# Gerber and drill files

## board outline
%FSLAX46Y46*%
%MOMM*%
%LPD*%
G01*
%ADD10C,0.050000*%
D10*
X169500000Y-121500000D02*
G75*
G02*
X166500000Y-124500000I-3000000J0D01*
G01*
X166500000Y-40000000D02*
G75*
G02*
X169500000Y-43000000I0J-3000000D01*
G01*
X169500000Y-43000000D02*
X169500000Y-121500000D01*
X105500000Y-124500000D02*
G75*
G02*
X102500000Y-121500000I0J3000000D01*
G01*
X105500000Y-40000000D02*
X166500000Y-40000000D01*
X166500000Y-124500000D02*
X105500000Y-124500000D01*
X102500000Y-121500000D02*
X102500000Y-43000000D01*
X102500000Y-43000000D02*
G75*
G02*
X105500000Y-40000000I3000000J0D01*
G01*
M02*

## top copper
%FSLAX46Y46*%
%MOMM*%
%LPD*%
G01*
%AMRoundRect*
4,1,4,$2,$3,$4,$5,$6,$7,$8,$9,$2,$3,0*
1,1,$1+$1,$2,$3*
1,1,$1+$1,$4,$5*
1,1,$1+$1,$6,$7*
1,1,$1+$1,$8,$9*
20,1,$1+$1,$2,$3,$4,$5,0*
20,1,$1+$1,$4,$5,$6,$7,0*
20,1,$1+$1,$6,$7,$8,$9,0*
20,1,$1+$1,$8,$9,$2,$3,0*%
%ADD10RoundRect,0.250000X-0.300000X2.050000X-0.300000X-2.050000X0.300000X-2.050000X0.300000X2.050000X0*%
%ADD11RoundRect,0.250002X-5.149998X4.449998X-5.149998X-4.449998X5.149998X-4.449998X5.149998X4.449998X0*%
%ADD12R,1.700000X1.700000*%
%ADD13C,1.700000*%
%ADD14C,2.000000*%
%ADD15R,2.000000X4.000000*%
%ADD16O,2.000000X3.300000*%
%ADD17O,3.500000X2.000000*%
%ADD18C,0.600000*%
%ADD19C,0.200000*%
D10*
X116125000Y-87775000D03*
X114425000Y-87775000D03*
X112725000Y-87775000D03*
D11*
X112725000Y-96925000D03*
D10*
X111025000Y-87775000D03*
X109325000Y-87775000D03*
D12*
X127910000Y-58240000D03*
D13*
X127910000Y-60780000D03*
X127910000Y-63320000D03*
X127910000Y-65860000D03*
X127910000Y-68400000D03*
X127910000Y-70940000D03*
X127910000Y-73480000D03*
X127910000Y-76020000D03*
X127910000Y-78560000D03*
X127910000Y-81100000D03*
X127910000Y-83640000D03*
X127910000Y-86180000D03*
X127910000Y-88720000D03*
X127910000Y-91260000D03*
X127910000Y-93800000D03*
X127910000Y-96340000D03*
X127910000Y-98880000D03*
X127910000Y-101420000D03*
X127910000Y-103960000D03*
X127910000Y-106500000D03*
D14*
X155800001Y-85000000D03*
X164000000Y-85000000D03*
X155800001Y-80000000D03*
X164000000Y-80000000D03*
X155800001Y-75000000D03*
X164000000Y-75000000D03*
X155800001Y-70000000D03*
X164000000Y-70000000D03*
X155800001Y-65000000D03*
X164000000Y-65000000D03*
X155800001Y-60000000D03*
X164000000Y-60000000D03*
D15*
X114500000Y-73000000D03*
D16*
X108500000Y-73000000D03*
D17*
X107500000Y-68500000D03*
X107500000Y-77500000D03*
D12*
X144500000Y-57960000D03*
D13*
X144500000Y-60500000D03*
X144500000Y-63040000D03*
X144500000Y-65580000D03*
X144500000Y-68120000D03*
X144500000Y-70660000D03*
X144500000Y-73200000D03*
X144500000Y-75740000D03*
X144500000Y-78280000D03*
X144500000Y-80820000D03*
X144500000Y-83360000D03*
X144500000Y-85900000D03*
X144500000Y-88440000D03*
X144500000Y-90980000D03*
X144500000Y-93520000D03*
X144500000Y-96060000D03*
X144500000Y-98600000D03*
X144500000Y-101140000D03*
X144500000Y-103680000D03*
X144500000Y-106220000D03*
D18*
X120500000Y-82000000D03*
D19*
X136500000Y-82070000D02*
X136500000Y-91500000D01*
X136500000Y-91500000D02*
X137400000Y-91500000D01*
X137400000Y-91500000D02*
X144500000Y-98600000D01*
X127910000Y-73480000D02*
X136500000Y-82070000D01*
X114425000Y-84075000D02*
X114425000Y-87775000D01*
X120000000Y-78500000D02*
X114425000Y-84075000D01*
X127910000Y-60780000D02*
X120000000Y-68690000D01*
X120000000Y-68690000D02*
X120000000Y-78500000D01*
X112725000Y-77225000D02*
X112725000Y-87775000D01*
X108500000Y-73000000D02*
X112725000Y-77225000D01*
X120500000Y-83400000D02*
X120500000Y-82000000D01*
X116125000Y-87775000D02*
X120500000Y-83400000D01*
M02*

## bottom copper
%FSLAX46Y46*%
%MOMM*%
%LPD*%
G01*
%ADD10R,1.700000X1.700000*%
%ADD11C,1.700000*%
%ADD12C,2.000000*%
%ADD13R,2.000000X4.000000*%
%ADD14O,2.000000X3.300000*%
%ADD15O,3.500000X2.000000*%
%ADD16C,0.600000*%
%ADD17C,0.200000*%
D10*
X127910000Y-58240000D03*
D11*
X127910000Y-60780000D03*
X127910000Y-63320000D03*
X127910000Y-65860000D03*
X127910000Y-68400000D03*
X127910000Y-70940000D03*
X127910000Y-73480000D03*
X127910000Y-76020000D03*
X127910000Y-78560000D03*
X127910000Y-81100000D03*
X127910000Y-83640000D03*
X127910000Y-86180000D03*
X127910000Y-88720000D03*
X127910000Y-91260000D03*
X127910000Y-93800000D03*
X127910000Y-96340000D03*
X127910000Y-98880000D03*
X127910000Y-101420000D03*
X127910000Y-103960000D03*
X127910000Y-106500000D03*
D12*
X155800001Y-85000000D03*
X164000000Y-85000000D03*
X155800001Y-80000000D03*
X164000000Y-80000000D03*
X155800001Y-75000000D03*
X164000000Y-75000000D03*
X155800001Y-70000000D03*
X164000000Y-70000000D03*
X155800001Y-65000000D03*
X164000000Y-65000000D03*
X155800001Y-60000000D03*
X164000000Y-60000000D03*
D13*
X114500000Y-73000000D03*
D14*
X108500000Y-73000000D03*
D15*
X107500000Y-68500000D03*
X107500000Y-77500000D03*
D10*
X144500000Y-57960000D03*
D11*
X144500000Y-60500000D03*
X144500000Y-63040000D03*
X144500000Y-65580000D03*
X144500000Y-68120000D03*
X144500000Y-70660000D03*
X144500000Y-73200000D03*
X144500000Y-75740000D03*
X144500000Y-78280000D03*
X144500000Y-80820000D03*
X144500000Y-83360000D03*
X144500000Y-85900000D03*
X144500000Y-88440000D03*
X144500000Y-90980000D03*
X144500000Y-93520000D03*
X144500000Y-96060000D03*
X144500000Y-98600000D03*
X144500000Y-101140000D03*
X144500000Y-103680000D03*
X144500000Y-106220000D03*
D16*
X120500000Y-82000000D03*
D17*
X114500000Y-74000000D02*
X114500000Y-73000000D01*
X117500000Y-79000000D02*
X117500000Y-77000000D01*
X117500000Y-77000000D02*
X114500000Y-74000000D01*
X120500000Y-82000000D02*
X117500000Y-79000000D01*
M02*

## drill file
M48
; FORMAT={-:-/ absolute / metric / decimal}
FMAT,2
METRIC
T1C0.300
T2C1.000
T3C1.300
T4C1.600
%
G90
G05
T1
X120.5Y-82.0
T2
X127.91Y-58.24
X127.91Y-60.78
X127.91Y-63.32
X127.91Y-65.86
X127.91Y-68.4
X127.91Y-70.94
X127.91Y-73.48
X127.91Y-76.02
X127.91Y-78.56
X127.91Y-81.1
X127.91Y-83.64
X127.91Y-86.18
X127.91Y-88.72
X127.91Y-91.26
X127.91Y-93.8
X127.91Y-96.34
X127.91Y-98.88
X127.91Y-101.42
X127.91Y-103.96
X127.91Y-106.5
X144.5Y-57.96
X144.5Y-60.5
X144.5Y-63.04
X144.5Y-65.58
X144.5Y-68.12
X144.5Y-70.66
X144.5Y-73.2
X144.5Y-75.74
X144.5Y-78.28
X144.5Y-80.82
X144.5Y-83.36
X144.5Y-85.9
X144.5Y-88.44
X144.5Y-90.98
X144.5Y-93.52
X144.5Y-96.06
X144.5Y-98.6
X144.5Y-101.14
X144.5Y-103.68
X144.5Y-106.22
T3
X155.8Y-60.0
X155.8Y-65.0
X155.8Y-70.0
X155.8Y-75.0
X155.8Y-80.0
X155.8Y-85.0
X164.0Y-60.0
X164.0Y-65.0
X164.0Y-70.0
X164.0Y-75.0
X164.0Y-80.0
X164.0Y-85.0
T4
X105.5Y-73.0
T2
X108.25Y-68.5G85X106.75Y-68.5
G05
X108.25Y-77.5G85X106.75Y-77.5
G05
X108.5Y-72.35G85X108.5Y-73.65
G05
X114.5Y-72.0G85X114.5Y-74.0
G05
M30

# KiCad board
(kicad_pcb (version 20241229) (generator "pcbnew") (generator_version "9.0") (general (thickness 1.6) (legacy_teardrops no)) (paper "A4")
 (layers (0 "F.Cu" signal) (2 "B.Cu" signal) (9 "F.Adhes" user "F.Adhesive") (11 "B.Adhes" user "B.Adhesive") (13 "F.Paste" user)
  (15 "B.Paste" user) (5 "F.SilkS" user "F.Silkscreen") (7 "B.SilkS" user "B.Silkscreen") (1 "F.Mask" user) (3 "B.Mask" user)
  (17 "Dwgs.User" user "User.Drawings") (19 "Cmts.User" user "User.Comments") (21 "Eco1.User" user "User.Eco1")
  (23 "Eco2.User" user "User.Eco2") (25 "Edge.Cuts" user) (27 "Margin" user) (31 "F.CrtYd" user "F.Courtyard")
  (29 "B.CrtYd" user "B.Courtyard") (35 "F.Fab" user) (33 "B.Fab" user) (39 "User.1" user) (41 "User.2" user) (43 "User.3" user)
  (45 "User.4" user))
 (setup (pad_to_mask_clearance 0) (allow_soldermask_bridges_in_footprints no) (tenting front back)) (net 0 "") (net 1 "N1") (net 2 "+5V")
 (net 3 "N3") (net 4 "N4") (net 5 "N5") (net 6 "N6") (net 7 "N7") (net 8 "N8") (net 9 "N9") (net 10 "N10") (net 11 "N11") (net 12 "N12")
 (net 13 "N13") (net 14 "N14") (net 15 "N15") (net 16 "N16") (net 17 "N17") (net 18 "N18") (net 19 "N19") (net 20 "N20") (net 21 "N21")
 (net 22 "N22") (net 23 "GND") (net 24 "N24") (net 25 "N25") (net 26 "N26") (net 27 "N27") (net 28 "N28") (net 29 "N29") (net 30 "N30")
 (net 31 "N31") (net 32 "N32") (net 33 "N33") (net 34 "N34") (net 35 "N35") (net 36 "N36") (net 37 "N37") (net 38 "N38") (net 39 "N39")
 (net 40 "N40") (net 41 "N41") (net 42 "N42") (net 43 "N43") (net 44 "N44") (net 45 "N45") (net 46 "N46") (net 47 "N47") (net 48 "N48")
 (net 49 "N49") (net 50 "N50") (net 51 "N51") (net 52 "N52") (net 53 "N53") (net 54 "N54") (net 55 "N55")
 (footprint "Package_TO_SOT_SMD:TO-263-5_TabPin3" (layer "F.Cu") (at 112.725 95.425 -90)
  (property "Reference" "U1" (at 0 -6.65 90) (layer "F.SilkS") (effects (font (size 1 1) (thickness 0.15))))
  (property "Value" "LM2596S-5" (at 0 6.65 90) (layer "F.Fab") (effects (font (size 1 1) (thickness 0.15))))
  (pad "" smd roundrect (at -0.925 -2.775 270) (size 4.55 5.25) (layers "F.Paste") (roundrect_rratio 0.054945))
  (pad "" smd roundrect (at -0.925 2.775 270) (size 4.55 5.25) (layers "F.Paste") (roundrect_rratio 0.054945))
  (pad "" smd roundrect (at 3.925 -2.775 270) (size 4.55 5.25) (layers "F.Paste") (roundrect_rratio 0.054945))
  (pad "" smd roundrect (at 3.925 2.775 270) (size 4.55 5.25) (layers "F.Paste") (roundrect_rratio 0.054945))
  (pad "1" smd roundrect (at -7.65 -3.4 270) (size 4.6 1.1) (layers "F.Cu" "F.Mask" "F.Paste") (roundrect_rratio 0.227273) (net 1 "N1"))
  (pad "2" smd roundrect (at -7.65 -1.7 270) (size 4.6 1.1) (layers "F.Cu" "F.Mask" "F.Paste") (roundrect_rratio 0.227273) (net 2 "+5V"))
  (pad "3" smd roundrect (at -7.65 0 270) (size 4.6 1.1) (layers "F.Cu" "F.Mask" "F.Paste") (roundrect_rratio 0.227273) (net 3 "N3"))
  (pad "3" smd roundrect (at 1.5 0 270) (size 9.4 10.8) (layers "F.Cu" "F.Mask") (roundrect_rratio 0.026596) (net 3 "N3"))
  (pad "4" smd roundrect (at -7.65 1.7 270) (size 4.6 1.1) (layers "F.Cu" "F.Mask" "F.Paste") (roundrect_rratio 0.227273) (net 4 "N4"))
  (pad "5" smd roundrect (at -7.65 3.4 270) (size 4.6 1.1) (layers "F.Cu" "F.Mask" "F.Paste") (roundrect_rratio 0.227273) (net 1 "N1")))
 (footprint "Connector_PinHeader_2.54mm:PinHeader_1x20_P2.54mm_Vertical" (layer "F.Cu") (at 127.91 58.24)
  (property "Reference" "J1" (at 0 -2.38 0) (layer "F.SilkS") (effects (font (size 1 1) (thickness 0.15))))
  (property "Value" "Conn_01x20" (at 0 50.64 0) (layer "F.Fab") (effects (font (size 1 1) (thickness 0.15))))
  (pad "1" thru_hole rect (at 0 0) (size 1.7 1.7) (drill 1) (layers "*.Cu" "*.Mask") (remove_unused_layers no) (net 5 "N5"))
  (pad "2" thru_hole circle (at 0 2.54) (size 1.7 1.7) (drill 1) (layers "*.Cu" "*.Mask") (remove_unused_layers no) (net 2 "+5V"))
  (pad "3" thru_hole circle (at 0 5.08) (size 1.7 1.7) (drill 1) (layers "*.Cu" "*.Mask") (remove_unused_layers no) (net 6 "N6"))
  (pad "4" thru_hole circle (at 0 7.62) (size 1.7 1.7) (drill 1) (layers "*.Cu" "*.Mask") (remove_unused_layers no) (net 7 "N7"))
  (pad "5" thru_hole circle (at 0 10.16) (size 1.7 1.7) (drill 1) (layers "*.Cu" "*.Mask") (remove_unused_layers no) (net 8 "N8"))
  (pad "6" thru_hole circle (at 0 12.7) (size 1.7 1.7) (drill 1) (layers "*.Cu" "*.Mask") (remove_unused_layers no) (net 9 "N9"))
  (pad "7" thru_hole circle (at 0 15.24) (size 1.7 1.7) (drill 1) (layers "*.Cu" "*.Mask") (remove_unused_layers no) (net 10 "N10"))
  (pad "8" thru_hole circle (at 0 17.78) (size 1.7 1.7) (drill 1) (layers "*.Cu" "*.Mask") (remove_unused_layers no) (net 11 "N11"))
  (pad "9" thru_hole circle (at 0 20.32) (size 1.7 1.7) (drill 1) (layers "*.Cu" "*.Mask") (remove_unused_layers no) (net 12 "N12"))
  (pad "10" thru_hole circle (at 0 22.86) (size 1.7 1.7) (drill 1) (layers "*.Cu" "*.Mask") (remove_unused_layers no) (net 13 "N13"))
  (pad "11" thru_hole circle (at 0 25.4) (size 1.7 1.7) (drill 1) (layers "*.Cu" "*.Mask") (remove_unused_layers no) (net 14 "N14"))
  (pad "12" thru_hole circle (at 0 27.94) (size 1.7 1.7) (drill 1) (layers "*.Cu" "*.Mask") (remove_unused_layers no) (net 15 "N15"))
  (pad "13" thru_hole circle (at 0 30.48) (size 1.7 1.7) (drill 1) (layers "*.Cu" "*.Mask") (remove_unused_layers no) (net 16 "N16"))
  (pad "14" thru_hole circle (at 0 33.02) (size 1.7 1.7) (drill 1) (layers "*.Cu" "*.Mask") (remove_unused_layers no) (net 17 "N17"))
  (pad "15" thru_hole circle (at 0 35.56) (size 1.7 1.7) (drill 1) (layers "*.Cu" "*.Mask") (remove_unused_layers no) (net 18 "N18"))
  (pad "16" thru_hole circle (at 0 38.1) (size 1.7 1.7) (drill 1) (layers "*.Cu" "*.Mask") (remove_unused_layers no) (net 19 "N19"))
  (pad "17" thru_hole circle (at 0 40.64) (size 1.7 1.7) (drill 1) (layers "*.Cu" "*.Mask") (remove_unused_layers no) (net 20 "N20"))
  (pad "18" thru_hole circle (at 0 43.18) (size 1.7 1.7) (drill 1) (layers "*.Cu" "*.Mask") (remove_unused_layers no) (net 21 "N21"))
  (pad "19" thru_hole circle (at 0 45.72) (size 1.7 1.7) (drill 1) (layers "*.Cu" "*.Mask") (remove_unused_layers no) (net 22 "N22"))
  (pad "20" thru_hole circle (at 0 48.26) (size 1.7 1.7) (drill 1) (layers "*.Cu" "*.Mask") (remove_unused_layers no) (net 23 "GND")))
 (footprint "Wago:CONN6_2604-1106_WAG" (layer "F.Cu") (at 155.800001 85 90)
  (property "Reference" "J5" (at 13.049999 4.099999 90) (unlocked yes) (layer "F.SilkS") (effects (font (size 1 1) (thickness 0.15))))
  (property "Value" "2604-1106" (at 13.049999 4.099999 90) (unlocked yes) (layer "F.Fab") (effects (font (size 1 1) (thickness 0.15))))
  (pad "1" thru_hole circle (at 0 0 90) (size 2 2) (drill 1.3) (layers "*.Cu" "*.Mask") (remove_unused_layers no) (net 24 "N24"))
  (pad "2" thru_hole circle (at 0 8.199999 90) (size 2 2) (drill 1.3) (layers "*.Cu" "*.Mask") (remove_unused_layers no) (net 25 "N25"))
  (pad "3" thru_hole circle (at 5 0 90) (size 2 2) (drill 1.3) (layers "*.Cu" "*.Mask") (remove_unused_layers no) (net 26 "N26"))
  (pad "4" thru_hole circle (at 5 8.199999 90) (size 2 2) (drill 1.3) (layers "*.Cu" "*.Mask") (remove_unused_layers no) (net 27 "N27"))
  (pad "5" thru_hole circle (at 10 0 90) (size 2 2) (drill 1.3) (layers "*.Cu" "*.Mask") (remove_unused_layers no) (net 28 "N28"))
  (pad "6" thru_hole circle (at 10 8.199999 90) (size 2 2) (drill 1.3) (layers "*.Cu" "*.Mask") (remove_unused_layers no) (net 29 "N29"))
  (pad "7" thru_hole circle (at 15 0 90) (size 2 2) (drill 1.3) (layers "*.Cu" "*.Mask") (remove_unused_layers no) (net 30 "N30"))
  (pad "8" thru_hole circle (at 15 8.199999 90) (size 2 2) (drill 1.3) (layers "*.Cu" "*.Mask") (remove_unused_layers no) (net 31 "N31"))
  (pad "9" thru_hole circle (at 20 0 90) (size 2 2) (drill 1.3) (layers "*.Cu" "*.Mask") (remove_unused_layers no) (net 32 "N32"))
  (pad "10" thru_hole circle (at 20 8.199999 90) (size 2 2) (drill 1.3) (layers "*.Cu" "*.Mask") (remove_unused_layers no) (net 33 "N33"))
  (pad "11" thru_hole circle (at 25 0 90) (size 2 2) (drill 1.3) (layers "*.Cu" "*.Mask") (remove_unused_layers no) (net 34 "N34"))
  (pad "12" thru_hole circle (at 25 8.199999 90) (size 2 2) (drill 1.3) (layers "*.Cu" "*.Mask") (remove_unused_layers no) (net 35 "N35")))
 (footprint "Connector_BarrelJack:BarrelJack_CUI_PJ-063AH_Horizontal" (layer "F.Cu") (at 114.5 73 -90)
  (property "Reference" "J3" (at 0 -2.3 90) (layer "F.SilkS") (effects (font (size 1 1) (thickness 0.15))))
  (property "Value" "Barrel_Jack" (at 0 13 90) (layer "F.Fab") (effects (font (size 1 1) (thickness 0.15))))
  (pad "" np_thru_hole circle (at 0 9 270) (size 1.6 1.6) (drill 1.6) (layers "*.Cu" "*.Mask"))
  (pad "1" thru_hole rect (at 0 0 270) (size 4 2) (drill oval 3 1) (layers "*.Cu" "*.Mask") (remove_unused_layers no) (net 1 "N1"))
  (pad "2" thru_hole oval (at 0 6 270) (size 3.3 2) (drill oval 2.3 1) (layers "*.Cu" "*.Mask") (remove_unused_layers no) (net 3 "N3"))
  (pad "MP" thru_hole oval (at -4.5 7 270) (size 2 3.5) (drill oval 1 2.5) (layers "*.Cu" "*.Mask") (remove_unused_layers no))
  (pad "MP" thru_hole oval (at 4.5 7 270) (size 2 3.5) (drill oval 1 2.5) (layers "*.Cu" "*.Mask") (remove_unused_layers no)))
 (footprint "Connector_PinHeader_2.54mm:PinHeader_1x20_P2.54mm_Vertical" (layer "F.Cu") (at 144.5 57.96)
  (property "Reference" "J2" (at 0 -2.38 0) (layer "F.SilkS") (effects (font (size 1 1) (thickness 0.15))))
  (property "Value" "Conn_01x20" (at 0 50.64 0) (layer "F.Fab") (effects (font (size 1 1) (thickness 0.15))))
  (pad "1" thru_hole rect (at 0 0) (size 1.7 1.7) (drill 1) (layers "*.Cu" "*.Mask") (remove_unused_layers no) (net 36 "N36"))
  (pad "2" thru_hole circle (at 0 2.54) (size 1.7 1.7) (drill 1) (layers "*.Cu" "*.Mask") (remove_unused_layers no) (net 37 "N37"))
  (pad "3" thru_hole circle (at 0 5.08) (size 1.7 1.7) (drill 1) (layers "*.Cu" "*.Mask") (remove_unused_layers no) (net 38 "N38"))
  (pad "4" thru_hole circle (at 0 7.62) (size 1.7 1.7) (drill 1) (layers "*.Cu" "*.Mask") (remove_unused_layers no) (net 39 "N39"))
  (pad "5" thru_hole circle (at 0 10.16) (size 1.7 1.7) (drill 1) (layers "*.Cu" "*.Mask") (remove_unused_layers no) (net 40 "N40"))
  (pad "6" thru_hole circle (at 0 12.7) (size 1.7 1.7) (drill 1) (layers "*.Cu" "*.Mask") (remove_unused_layers no) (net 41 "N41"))
  (pad "7" thru_hole circle (at 0 15.24) (size 1.7 1.7) (drill 1) (layers "*.Cu" "*.Mask") (remove_unused_layers no) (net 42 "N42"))
  (pad "8" thru_hole circle (at 0 17.78) (size 1.7 1.7) (drill 1) (layers "*.Cu" "*.Mask") (remove_unused_layers no) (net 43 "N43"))
  (pad "9" thru_hole circle (at 0 20.32) (size 1.7 1.7) (drill 1) (layers "*.Cu" "*.Mask") (remove_unused_layers no) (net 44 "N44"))
  (pad "10" thru_hole circle (at 0 22.86) (size 1.7 1.7) (drill 1) (layers "*.Cu" "*.Mask") (remove_unused_layers no) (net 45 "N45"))
  (pad "11" thru_hole circle (at 0 25.4) (size 1.7 1.7) (drill 1) (layers "*.Cu" "*.Mask") (remove_unused_layers no) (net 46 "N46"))
  (pad "12" thru_hole circle (at 0 27.94) (size 1.7 1.7) (drill 1) (layers "*.Cu" "*.Mask") (remove_unused_layers no) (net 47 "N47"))
  (pad "13" thru_hole circle (at 0 30.48) (size 1.7 1.7) (drill 1) (layers "*.Cu" "*.Mask") (remove_unused_layers no) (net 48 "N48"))
  (pad "14" thru_hole circle (at 0 33.02) (size 1.7 1.7) (drill 1) (layers "*.Cu" "*.Mask") (remove_unused_layers no) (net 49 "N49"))
  (pad "15" thru_hole circle (at 0 35.56) (size 1.7 1.7) (drill 1) (layers "*.Cu" "*.Mask") (remove_unused_layers no) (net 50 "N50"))
  (pad "16" thru_hole circle (at 0 38.1) (size 1.7 1.7) (drill 1) (layers "*.Cu" "*.Mask") (remove_unused_layers no) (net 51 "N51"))
  (pad "17" thru_hole circle (at 0 40.64) (size 1.7 1.7) (drill 1) (layers "*.Cu" "*.Mask") (remove_unused_layers no) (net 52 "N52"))
  (pad "18" thru_hole circle (at 0 43.18) (size 1.7 1.7) (drill 1) (layers "*.Cu" "*.Mask") (remove_unused_layers no) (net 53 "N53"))
  (pad "19" thru_hole circle (at 0 45.72) (size 1.7 1.7) (drill 1) (layers "*.Cu" "*.Mask") (remove_unused_layers no) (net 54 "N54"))
  (pad "20" thru_hole circle (at 0 48.26) (size 1.7 1.7) (drill 1) (layers "*.Cu" "*.Mask") (remove_unused_layers no) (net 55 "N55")))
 (gr_arc (start 169.5 121.5) (mid 168.62132 123.62132) (end 166.5 124.5) (stroke (width 0.05) (type default)) (layer "Edge.Cuts"))
 (gr_arc (start 166.5 40) (mid 168.62132 40.87868) (end 169.5 43) (stroke (width 0.05) (type default)) (layer "Edge.Cuts"))
 (gr_line (start 169.5 43) (end 169.5 121.5) (stroke (width 0.05) (type default)) (layer "Edge.Cuts"))
 (gr_arc (start 105.5 124.5) (mid 103.37868 123.62132) (end 102.5 121.5) (stroke (width 0.05) (type default)) (layer "Edge.Cuts"))
 (gr_line (start 105.5 40) (end 166.5 40) (stroke (width 0.05) (type default)) (layer "Edge.Cuts"))
 (gr_line (start 166.5 124.5) (end 105.5 124.5) (stroke (width 0.05) (type default)) (layer "Edge.Cuts"))
 (gr_line (start 102.5 121.5) (end 102.5 43) (stroke (width 0.05) (type default)) (layer "Edge.Cuts"))
 (gr_arc (start 102.5 43) (mid 103.37868 40.87868) (end 105.5 40) (stroke (width 0.05) (type default)) (layer "Edge.Cuts"))
 (segment (start 136.5 82.07) (end 136.5 91.5) (width 0.2) (layer "F.Cu") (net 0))
 (segment (start 136.5 91.5) (end 137.4 91.5) (width 0.2) (layer "F.Cu") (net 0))
 (segment (start 137.4 91.5) (end 144.5 98.6) (width 0.2) (layer "F.Cu") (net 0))
 (segment (start 127.91 73.48) (end 136.5 82.07) (width 0.2) (layer "F.Cu") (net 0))
 (segment (start 114.425 84.075) (end 114.425 87.775) (width 0.2) (layer "F.Cu") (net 2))
 (segment (start 120 78.5) (end 114.425 84.075) (width 0.2) (layer "F.Cu") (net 2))
 (segment (start 127.91 60.78) (end 120 68.69) (width 0.2) (layer "F.Cu") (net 2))
 (segment (start 120 68.69) (end 120 78.5) (width 0.2) (layer "F.Cu") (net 2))
 (segment (start 112.725 77.225) (end 112.725 87.775) (width 0.2) (layer "F.Cu") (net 3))
 (segment (start 108.5 73) (end 112.725 77.225) (width 0.2) (layer "F.Cu") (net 3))
 (segment (start 120.5 83.4) (end 120.5 82) (width 0.2) (layer "F.Cu") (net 1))
 (segment (start 116.125 87.775) (end 120.5 83.4) (width 0.2) (layer "F.Cu") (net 1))
 (via (at 120.5 82) (size 0.6) (drill 0.3) (layers "F.Cu" "B.Cu") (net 1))
 (segment (start 114.5 74) (end 114.5 73) (width 0.2) (layer "B.Cu") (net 1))
 (segment (start 117.5 79) (end 117.5 77) (width 0.2) (layer "B.Cu") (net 1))
 (segment (start 117.5 77) (end 114.5 74) (width 0.2) (layer "B.Cu") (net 1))
 (segment (start 120.5 82) (end 117.5 79) (width 0.2) (layer "B.Cu") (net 1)))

